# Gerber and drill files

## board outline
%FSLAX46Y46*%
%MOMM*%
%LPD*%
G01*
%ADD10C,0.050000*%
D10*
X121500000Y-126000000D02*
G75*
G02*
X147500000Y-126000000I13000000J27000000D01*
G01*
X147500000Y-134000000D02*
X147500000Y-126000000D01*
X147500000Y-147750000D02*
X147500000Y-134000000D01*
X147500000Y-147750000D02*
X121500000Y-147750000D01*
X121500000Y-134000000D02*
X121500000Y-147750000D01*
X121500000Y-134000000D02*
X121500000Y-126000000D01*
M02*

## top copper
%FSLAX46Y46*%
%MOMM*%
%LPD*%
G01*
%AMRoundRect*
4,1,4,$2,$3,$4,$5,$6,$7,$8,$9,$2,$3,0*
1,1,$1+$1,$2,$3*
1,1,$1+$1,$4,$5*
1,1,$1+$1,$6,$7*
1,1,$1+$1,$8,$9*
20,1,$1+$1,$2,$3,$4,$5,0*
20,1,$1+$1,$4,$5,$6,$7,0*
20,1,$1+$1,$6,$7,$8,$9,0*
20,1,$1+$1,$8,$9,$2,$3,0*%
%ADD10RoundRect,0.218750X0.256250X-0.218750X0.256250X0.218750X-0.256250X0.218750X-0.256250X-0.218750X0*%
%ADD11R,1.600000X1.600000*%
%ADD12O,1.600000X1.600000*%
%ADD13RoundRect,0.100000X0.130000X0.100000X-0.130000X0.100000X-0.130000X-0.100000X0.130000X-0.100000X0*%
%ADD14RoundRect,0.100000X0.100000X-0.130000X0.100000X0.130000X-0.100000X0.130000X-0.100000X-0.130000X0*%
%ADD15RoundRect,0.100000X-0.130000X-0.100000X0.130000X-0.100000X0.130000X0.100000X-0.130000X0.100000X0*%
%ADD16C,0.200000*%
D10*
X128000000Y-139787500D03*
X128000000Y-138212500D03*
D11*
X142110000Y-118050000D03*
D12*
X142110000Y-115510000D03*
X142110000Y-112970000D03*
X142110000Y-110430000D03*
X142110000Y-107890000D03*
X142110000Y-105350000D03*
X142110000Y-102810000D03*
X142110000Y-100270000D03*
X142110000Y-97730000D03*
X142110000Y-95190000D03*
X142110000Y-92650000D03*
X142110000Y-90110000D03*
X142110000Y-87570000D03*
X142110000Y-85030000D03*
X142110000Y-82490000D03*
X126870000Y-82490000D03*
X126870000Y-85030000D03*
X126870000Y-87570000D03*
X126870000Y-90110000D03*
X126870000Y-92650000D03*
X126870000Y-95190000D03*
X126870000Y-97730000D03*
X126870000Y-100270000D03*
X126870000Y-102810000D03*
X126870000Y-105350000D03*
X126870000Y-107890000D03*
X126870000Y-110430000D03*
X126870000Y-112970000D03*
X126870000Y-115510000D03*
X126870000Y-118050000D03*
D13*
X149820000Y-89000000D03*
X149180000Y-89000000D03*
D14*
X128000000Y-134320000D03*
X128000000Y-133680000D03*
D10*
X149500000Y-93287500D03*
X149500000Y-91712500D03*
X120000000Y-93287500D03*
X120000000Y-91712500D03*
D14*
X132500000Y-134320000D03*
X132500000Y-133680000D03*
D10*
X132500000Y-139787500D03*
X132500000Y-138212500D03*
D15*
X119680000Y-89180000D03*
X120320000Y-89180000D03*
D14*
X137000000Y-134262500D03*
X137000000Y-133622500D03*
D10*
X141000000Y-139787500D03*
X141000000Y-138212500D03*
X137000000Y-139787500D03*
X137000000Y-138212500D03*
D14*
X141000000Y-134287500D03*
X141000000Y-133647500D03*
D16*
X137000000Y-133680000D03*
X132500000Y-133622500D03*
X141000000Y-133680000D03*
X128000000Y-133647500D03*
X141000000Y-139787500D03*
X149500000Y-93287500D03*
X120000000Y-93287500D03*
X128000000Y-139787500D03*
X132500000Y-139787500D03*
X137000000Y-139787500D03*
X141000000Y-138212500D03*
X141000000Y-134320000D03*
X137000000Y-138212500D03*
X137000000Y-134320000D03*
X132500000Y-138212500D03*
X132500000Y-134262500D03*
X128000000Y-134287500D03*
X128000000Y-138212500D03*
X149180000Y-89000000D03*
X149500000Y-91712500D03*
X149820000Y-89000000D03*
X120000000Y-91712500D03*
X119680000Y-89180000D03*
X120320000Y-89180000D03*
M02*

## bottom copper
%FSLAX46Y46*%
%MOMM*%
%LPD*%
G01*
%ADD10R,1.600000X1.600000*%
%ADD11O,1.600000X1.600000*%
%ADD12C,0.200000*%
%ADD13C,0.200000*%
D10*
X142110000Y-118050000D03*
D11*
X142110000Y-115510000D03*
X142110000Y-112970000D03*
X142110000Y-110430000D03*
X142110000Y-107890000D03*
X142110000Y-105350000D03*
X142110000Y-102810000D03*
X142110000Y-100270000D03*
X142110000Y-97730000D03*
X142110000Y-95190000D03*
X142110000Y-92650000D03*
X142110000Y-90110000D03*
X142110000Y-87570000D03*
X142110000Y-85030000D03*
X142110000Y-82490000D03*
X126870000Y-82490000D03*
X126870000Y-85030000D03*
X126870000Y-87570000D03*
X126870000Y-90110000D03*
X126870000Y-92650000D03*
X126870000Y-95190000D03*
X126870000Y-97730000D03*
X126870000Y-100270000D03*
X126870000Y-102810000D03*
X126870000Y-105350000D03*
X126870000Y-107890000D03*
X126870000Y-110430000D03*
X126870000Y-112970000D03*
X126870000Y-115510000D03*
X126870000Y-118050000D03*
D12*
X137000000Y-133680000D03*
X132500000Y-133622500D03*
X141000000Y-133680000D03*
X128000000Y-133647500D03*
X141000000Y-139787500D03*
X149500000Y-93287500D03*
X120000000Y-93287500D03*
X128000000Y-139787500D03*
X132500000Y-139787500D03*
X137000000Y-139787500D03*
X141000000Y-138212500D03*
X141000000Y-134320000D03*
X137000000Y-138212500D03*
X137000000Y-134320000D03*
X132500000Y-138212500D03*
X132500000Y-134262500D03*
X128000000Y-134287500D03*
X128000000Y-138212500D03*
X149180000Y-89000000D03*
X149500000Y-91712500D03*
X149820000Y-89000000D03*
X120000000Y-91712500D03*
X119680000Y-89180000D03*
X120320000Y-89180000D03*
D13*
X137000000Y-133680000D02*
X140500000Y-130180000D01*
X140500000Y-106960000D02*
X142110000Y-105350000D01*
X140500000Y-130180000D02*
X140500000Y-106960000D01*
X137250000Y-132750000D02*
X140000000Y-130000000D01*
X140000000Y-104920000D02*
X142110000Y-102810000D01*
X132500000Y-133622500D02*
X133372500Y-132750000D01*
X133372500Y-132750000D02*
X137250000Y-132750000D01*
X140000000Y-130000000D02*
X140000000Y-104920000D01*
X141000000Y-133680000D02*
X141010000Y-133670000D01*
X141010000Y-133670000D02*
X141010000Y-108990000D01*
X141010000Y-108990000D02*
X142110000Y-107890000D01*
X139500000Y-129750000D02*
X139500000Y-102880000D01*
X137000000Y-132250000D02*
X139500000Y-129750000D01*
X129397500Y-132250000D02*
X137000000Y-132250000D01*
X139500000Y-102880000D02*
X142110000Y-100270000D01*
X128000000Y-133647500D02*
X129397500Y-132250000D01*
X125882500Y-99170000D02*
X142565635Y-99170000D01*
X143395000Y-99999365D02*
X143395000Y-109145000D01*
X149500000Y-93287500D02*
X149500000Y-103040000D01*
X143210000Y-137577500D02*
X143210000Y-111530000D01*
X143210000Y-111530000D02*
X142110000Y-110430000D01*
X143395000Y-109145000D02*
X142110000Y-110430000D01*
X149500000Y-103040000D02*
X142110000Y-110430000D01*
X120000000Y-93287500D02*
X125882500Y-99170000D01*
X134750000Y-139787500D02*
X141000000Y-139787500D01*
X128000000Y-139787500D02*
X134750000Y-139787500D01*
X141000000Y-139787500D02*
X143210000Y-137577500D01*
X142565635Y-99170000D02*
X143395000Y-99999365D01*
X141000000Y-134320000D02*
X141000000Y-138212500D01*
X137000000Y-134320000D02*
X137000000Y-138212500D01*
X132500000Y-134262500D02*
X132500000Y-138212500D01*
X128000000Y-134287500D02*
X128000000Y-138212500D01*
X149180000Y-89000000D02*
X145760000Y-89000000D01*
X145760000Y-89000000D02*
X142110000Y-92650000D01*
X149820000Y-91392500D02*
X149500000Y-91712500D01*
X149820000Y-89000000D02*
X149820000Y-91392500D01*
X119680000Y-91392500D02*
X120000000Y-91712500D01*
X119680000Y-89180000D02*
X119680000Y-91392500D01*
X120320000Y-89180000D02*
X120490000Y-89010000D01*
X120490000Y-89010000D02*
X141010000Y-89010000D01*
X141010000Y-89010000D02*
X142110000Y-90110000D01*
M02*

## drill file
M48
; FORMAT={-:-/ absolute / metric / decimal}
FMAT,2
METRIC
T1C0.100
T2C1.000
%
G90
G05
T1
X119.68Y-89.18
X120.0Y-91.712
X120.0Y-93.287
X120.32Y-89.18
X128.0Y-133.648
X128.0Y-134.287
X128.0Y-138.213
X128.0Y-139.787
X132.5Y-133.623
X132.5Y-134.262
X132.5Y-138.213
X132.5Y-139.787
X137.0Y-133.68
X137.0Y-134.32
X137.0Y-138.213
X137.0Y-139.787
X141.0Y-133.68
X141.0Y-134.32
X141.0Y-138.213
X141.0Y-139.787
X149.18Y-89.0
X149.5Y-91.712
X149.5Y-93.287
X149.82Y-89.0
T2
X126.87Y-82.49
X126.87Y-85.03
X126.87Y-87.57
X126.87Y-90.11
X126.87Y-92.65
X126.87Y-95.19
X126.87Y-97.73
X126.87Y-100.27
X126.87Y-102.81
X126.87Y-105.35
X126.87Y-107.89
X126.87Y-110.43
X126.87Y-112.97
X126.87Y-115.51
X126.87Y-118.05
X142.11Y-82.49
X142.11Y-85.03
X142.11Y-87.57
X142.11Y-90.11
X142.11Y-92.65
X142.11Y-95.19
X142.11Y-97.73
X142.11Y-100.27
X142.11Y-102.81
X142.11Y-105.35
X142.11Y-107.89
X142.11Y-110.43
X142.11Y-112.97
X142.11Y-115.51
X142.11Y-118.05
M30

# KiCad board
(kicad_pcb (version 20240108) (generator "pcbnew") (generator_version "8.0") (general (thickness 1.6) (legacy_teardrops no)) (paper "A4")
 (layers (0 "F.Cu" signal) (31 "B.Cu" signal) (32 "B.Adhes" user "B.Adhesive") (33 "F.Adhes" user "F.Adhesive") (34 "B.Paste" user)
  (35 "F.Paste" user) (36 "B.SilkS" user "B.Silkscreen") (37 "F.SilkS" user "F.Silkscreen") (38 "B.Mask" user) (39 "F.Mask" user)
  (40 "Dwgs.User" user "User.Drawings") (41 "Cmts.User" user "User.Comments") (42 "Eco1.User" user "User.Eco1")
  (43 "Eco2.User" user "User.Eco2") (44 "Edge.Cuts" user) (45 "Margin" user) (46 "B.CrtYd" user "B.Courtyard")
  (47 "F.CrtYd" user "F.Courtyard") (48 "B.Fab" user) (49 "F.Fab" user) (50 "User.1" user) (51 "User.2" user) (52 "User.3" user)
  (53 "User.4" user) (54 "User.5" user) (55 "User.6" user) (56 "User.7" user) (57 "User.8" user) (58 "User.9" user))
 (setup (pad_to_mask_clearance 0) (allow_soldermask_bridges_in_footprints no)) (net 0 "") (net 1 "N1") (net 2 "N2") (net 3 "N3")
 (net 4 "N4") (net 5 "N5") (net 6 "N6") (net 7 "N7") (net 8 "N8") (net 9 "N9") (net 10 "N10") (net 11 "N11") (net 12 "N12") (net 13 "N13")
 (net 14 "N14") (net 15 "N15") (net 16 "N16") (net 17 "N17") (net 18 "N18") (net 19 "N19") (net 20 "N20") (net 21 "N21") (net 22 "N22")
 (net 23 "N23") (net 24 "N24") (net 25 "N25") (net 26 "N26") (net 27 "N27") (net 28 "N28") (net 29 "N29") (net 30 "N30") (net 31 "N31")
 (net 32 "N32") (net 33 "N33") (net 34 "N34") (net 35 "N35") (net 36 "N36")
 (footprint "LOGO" (layer "F.Cu") (at 123.1 146.2)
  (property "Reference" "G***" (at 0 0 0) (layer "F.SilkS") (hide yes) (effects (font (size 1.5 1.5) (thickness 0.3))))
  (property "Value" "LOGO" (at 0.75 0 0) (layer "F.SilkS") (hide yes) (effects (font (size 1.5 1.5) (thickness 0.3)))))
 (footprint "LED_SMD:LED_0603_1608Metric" (layer "F.Cu") (at 128 139 90)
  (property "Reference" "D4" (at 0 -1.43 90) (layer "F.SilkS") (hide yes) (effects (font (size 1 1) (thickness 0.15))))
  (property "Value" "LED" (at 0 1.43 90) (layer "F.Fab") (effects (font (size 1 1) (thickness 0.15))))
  (pad "1" smd roundrect (at -0.7875 0 90) (size 0.875 0.95) (layers "F.Cu" "F.Paste" "F.Mask") (roundrect_rratio 0.25) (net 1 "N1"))
  (pad "2" smd roundrect (at 0.7875 0 90) (size 0.875 0.95) (layers "F.Cu" "F.Paste" "F.Mask") (roundrect_rratio 0.25) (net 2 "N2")))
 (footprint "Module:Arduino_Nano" (layer "F.Cu") (at 142.11 118.05 180)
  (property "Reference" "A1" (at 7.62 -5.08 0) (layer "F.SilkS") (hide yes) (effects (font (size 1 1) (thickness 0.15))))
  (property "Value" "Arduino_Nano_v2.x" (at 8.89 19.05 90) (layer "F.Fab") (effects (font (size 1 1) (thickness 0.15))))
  (pad "1" thru_hole rect (at 0 0 180) (size 1.6 1.6) (drill 1) (layers "*.Cu" "*.Mask") (remove_unused_layers no) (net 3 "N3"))
  (pad "2" thru_hole oval (at 0 2.54 180) (size 1.6 1.6) (drill 1) (layers "*.Cu" "*.Mask") (remove_unused_layers no) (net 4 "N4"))
  (pad "3" thru_hole oval (at 0 5.08 180) (size 1.6 1.6) (drill 1) (layers "*.Cu" "*.Mask") (remove_unused_layers no) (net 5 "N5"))
  (pad "4" thru_hole oval (at 0 7.62 180) (size 1.6 1.6) (drill 1) (layers "*.Cu" "*.Mask") (remove_unused_layers no) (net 1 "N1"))
  (pad "5" thru_hole oval (at 0 10.16 180) (size 1.6 1.6) (drill 1) (layers "*.Cu" "*.Mask") (remove_unused_layers no) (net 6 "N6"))
  (pad "6" thru_hole oval (at 0 12.7 180) (size 1.6 1.6) (drill 1) (layers "*.Cu" "*.Mask") (remove_unused_layers no) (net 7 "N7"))
  (pad "7" thru_hole oval (at 0 15.24 180) (size 1.6 1.6) (drill 1) (layers "*.Cu" "*.Mask") (remove_unused_layers no) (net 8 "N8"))
  (pad "8" thru_hole oval (at 0 17.78 180) (size 1.6 1.6) (drill 1) (layers "*.Cu" "*.Mask") (remove_unused_layers no) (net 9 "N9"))
  (pad "9" thru_hole oval (at 0 20.32 180) (size 1.6 1.6) (drill 1) (layers "*.Cu" "*.Mask") (remove_unused_layers no) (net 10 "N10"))
  (pad "10" thru_hole oval (at 0 22.86 180) (size 1.6 1.6) (drill 1) (layers "*.Cu" "*.Mask") (remove_unused_layers no) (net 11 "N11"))
  (pad "11" thru_hole oval (at 0 25.4 180) (size 1.6 1.6) (drill 1) (layers "*.Cu" "*.Mask") (remove_unused_layers no) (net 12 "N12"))
  (pad "12" thru_hole oval (at 0 27.94 180) (size 1.6 1.6) (drill 1) (layers "*.Cu" "*.Mask") (remove_unused_layers no) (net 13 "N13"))
  (pad "13" thru_hole oval (at 0 30.48 180) (size 1.6 1.6) (drill 1) (layers "*.Cu" "*.Mask") (remove_unused_layers no) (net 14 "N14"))
  (pad "14" thru_hole oval (at 0 33.02 180) (size 1.6 1.6) (drill 1) (layers "*.Cu" "*.Mask") (remove_unused_layers no) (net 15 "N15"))
  (pad "15" thru_hole oval (at 0 35.56 180) (size 1.6 1.6) (drill 1) (layers "*.Cu" "*.Mask") (remove_unused_layers no) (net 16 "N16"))
  (pad "16" thru_hole oval (at 15.24 35.56 180) (size 1.6 1.6) (drill 1) (layers "*.Cu" "*.Mask") (remove_unused_layers no) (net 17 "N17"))
  (pad "17" thru_hole oval (at 15.24 33.02 180) (size 1.6 1.6) (drill 1) (layers "*.Cu" "*.Mask") (remove_unused_layers no) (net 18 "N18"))
  (pad "18" thru_hole oval (at 15.24 30.48 180) (size 1.6 1.6) (drill 1) (layers "*.Cu" "*.Mask") (remove_unused_layers no) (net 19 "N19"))
  (pad "19" thru_hole oval (at 15.24 27.94 180) (size 1.6 1.6) (drill 1) (layers "*.Cu" "*.Mask") (remove_unused_layers no) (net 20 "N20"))
  (pad "20" thru_hole oval (at 15.24 25.4 180) (size 1.6 1.6) (drill 1) (layers "*.Cu" "*.Mask") (remove_unused_layers no) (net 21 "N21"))
  (pad "21" thru_hole oval (at 15.24 22.86 180) (size 1.6 1.6) (drill 1) (layers "*.Cu" "*.Mask") (remove_unused_layers no) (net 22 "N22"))
  (pad "22" thru_hole oval (at 15.24 20.32 180) (size 1.6 1.6) (drill 1) (layers "*.Cu" "*.Mask") (remove_unused_layers no) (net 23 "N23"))
  (pad "23" thru_hole oval (at 15.24 17.78 180) (size 1.6 1.6) (drill 1) (layers "*.Cu" "*.Mask") (remove_unused_layers no) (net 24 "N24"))
  (pad "24" thru_hole oval (at 15.24 15.24 180) (size 1.6 1.6) (drill 1) (layers "*.Cu" "*.Mask") (remove_unused_layers no) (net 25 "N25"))
  (pad "25" thru_hole oval (at 15.24 12.7 180) (size 1.6 1.6) (drill 1) (layers "*.Cu" "*.Mask") (remove_unused_layers no) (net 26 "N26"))
  (pad "26" thru_hole oval (at 15.24 10.16 180) (size 1.6 1.6) (drill 1) (layers "*.Cu" "*.Mask") (remove_unused_layers no) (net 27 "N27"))
  (pad "27" thru_hole oval (at 15.24 7.62 180) (size 1.6 1.6) (drill 1) (layers "*.Cu" "*.Mask") (remove_unused_layers no) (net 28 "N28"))
  (pad "28" thru_hole oval (at 15.24 5.08 180) (size 1.6 1.6) (drill 1) (layers "*.Cu" "*.Mask") (remove_unused_layers no) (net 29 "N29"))
  (pad "29" thru_hole oval (at 15.24 2.54 180) (size 1.6 1.6) (drill 1) (layers "*.Cu" "*.Mask") (remove_unused_layers no) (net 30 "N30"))
  (pad "30" thru_hole oval (at 15.24 0 180) (size 1.6 1.6) (drill 1) (layers "*.Cu" "*.Mask") (remove_unused_layers no) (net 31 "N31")))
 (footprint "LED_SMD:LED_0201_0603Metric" (layer "F.Cu") (at 149.5 89 180)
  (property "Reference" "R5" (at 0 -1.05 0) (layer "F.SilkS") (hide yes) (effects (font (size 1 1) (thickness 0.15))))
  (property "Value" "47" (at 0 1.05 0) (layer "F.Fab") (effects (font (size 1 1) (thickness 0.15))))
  (pad "" smd roundrect (at -0.345 0 180) (size 0.318 0.36) (layers "F.Paste") (roundrect_rratio 0.25))
  (pad "" smd roundrect (at 0.345 0 180) (size 0.318 0.36) (layers "F.Paste") (roundrect_rratio 0.25))
  (pad "1" smd roundrect (at -0.32 0 180) (size 0.46 0.4) (layers "F.Cu" "F.Mask") (roundrect_rratio 0.25) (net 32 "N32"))
  (pad "2" smd roundrect (at 0.32 0 180) (size 0.46 0.4) (layers "F.Cu" "F.Mask") (roundrect_rratio 0.25) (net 12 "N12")))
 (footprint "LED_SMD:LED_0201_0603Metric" (layer "F.Cu") (at 128 134 90)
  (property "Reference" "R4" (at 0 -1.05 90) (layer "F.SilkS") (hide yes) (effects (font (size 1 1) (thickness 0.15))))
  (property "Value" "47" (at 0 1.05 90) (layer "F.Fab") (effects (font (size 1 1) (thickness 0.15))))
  (pad "" smd roundrect (at -0.345 0 90) (size 0.318 0.36) (layers "F.Paste") (roundrect_rratio 0.25))
  (pad "" smd roundrect (at 0.345 0 90) (size 0.318 0.36) (layers "F.Paste") (roundrect_rratio 0.25))
  (pad "1" smd roundrect (at -0.32 0 90) (size 0.46 0.4) (layers "F.Cu" "F.Mask") (roundrect_rratio 0.25) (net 2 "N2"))
  (pad "2" smd roundrect (at 0.32 0 90) (size 0.46 0.4) (layers "F.Cu" "F.Mask") (roundrect_rratio 0.25) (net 9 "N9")))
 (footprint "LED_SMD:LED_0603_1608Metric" (layer "F.Cu") (at 149.5 92.5 90)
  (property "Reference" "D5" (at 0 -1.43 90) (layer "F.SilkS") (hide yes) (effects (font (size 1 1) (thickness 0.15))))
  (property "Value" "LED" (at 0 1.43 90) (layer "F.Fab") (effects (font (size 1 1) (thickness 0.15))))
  (pad "1" smd roundrect (at -0.7875 0 90) (size 0.875 0.95) (layers "F.Cu" "F.Paste" "F.Mask") (roundrect_rratio 0.25) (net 1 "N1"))
  (pad "2" smd roundrect (at 0.7875 0 90) (size 0.875 0.95) (layers "F.Cu" "F.Paste" "F.Mask") (roundrect_rratio 0.25) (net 32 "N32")))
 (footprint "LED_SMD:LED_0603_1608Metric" (layer "F.Cu") (at 120 92.5 90)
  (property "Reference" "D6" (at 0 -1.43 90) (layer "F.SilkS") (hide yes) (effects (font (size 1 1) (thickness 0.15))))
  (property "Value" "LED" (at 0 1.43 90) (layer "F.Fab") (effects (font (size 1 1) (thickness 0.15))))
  (pad "1" smd roundrect (at -0.7875 0 90) (size 0.875 0.95) (layers "F.Cu" "F.Paste" "F.Mask") (roundrect_rratio 0.25) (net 1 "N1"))
  (pad "2" smd roundrect (at 0.7875 0 90) (size 0.875 0.95) (layers "F.Cu" "F.Paste" "F.Mask") (roundrect_rratio 0.25) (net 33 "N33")))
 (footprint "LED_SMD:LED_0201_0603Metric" (layer "F.Cu") (at 132.5 134 90)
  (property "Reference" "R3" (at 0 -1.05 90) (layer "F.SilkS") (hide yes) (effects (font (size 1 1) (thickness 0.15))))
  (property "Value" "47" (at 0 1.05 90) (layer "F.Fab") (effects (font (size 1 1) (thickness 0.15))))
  (pad "" smd roundrect (at -0.345 0 90) (size 0.318 0.36) (layers "F.Paste") (roundrect_rratio 0.25))
  (pad "" smd roundrect (at 0.345 0 90) (size 0.318 0.36) (layers "F.Paste") (roundrect_rratio 0.25))
  (pad "1" smd roundrect (at -0.32 0 90) (size 0.46 0.4) (layers "F.Cu" "F.Mask") (roundrect_rratio 0.25) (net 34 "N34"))
  (pad "2" smd roundrect (at 0.32 0 90) (size 0.46 0.4) (layers "F.Cu" "F.Mask") (roundrect_rratio 0.25) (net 8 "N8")))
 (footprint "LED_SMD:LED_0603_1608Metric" (layer "F.Cu") (at 132.5 139 90)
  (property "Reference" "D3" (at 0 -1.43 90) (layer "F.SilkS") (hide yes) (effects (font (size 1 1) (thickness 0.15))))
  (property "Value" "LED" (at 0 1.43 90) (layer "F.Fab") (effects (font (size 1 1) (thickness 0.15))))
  (pad "1" smd roundrect (at -0.7875 0 90) (size 0.875 0.95) (layers "F.Cu" "F.Paste" "F.Mask") (roundrect_rratio 0.25) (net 1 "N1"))
  (pad "2" smd roundrect (at 0.7875 0 90) (size 0.875 0.95) (layers "F.Cu" "F.Paste" "F.Mask") (roundrect_rratio 0.25) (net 34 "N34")))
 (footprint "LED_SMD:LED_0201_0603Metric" (layer "F.Cu") (at 120 89.18)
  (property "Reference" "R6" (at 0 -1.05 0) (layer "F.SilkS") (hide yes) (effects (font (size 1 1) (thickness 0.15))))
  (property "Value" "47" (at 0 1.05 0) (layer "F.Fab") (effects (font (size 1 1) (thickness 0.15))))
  (pad "" smd roundrect (at -0.345 0) (size 0.318 0.36) (layers "F.Paste") (roundrect_rratio 0.25))
  (pad "" smd roundrect (at 0.345 0) (size 0.318 0.36) (layers "F.Paste") (roundrect_rratio 0.25))
  (pad "1" smd roundrect (at -0.32 0) (size 0.46 0.4) (layers "F.Cu" "F.Mask") (roundrect_rratio 0.25) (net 33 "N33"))
  (pad "2" smd roundrect (at 0.32 0) (size 0.46 0.4) (layers "F.Cu" "F.Mask") (roundrect_rratio 0.25) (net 13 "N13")))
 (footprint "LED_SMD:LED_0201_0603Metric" (layer "F.Cu") (at 137 133.9425 90)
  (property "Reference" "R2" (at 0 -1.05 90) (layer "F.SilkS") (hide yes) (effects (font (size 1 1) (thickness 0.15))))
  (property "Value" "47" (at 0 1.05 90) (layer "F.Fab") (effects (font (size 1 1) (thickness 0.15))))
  (pad "" smd roundrect (at -0.345 0 90) (size 0.318 0.36) (layers "F.Paste") (roundrect_rratio 0.25))
  (pad "" smd roundrect (at 0.345 0 90) (size 0.318 0.36) (layers "F.Paste") (roundrect_rratio 0.25))
  (pad "1" smd roundrect (at -0.32 0 90) (size 0.46 0.4) (layers "F.Cu" "F.Mask") (roundrect_rratio 0.25) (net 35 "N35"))
  (pad "2" smd roundrect (at 0.32 0 90) (size 0.46 0.4) (layers "F.Cu" "F.Mask") (roundrect_rratio 0.25) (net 7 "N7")))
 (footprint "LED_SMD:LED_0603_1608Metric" (layer "F.Cu") (at 141 139 90)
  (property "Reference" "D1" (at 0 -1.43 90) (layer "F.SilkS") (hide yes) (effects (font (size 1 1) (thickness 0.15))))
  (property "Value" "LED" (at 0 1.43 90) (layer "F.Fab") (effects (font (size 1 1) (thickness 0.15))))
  (pad "1" smd roundrect (at -0.7875 0 90) (size 0.875 0.95) (layers "F.Cu" "F.Paste" "F.Mask") (roundrect_rratio 0.25) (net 1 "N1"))
  (pad "2" smd roundrect (at 0.7875 0 90) (size 0.875 0.95) (layers "F.Cu" "F.Paste" "F.Mask") (roundrect_rratio 0.25) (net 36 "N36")))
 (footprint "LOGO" (layer "F.Cu") (at 134.5 115.75 90)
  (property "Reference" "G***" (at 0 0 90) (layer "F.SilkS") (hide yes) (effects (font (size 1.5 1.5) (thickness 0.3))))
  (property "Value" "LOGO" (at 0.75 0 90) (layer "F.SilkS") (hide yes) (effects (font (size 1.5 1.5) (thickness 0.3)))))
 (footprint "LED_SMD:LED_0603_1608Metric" (layer "F.Cu") (at 137 139 90)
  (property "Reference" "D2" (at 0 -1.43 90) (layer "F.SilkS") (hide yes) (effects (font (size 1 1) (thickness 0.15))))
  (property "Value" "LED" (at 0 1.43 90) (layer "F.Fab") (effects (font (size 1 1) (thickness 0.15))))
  (pad "1" smd roundrect (at -0.7875 0 90) (size 0.875 0.95) (layers "F.Cu" "F.Paste" "F.Mask") (roundrect_rratio 0.25) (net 1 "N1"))
  (pad "2" smd roundrect (at 0.7875 0 90) (size 0.875 0.95) (layers "F.Cu" "F.Paste" "F.Mask") (roundrect_rratio 0.25) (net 35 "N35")))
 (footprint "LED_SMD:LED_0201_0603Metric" (layer "F.Cu") (at 141 133.9675 90)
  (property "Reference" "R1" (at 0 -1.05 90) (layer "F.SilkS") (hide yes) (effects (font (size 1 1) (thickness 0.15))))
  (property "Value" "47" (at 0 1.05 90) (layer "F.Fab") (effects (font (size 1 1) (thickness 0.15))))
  (pad "" smd roundrect (at -0.345 0 90) (size 0.318 0.36) (layers "F.Paste") (roundrect_rratio 0.25))
  (pad "" smd roundrect (at 0.345 0 90) (size 0.318 0.36) (layers "F.Paste") (roundrect_rratio 0.25))
  (pad "1" smd roundrect (at -0.32 0 90) (size 0.46 0.4) (layers "F.Cu" "F.Mask") (roundrect_rratio 0.25) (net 36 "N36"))
  (pad "2" smd roundrect (at 0.32 0 90) (size 0.46 0.4) (layers "F.Cu" "F.Mask") (roundrect_rratio 0.25) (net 6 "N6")))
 (gr_arc (start 121.5 126) (mid 134.5 69.033352) (end 147.5 126) (stroke (width 0.05) (type default)) (layer "Edge.Cuts"))
 (gr_line (start 147.5 134) (end 147.5 126) (stroke (width 0.05) (type default)) (layer "Edge.Cuts"))
 (gr_line (start 147.5 147.75) (end 147.5 134) (stroke (width 0.05) (type default)) (layer "Edge.Cuts"))
 (gr_line (start 147.5 147.75) (end 121.5 147.75) (stroke (width 0.05) (type default)) (layer "Edge.Cuts"))
 (gr_line (start 121.5 134) (end 121.5 147.75) (stroke (width 0.05) (type default)) (layer "Edge.Cuts"))
 (gr_line (start 121.5 134) (end 121.5 126) (stroke (width 0.05) (type default)) (layer "Edge.Cuts"))
 (via (at 137 133.68) (size 0.2) (drill 0.1) (layers "F.Cu" "B.Cu") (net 7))
 (segment (start 137 133.68) (end 140.5 130.18) (width 0.2) (layer "B.Cu") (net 7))
 (segment (start 140.5 106.96) (end 142.11 105.35) (width 0.2) (layer "B.Cu") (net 7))
 (segment (start 140.5 130.18) (end 140.5 106.96) (width 0.2) (layer "B.Cu") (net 7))
 (via (at 132.5 133.6225) (size 0.2) (drill 0.1) (layers "F.Cu" "B.Cu") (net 8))
 (segment (start 137.25 132.75) (end 140 130) (width 0.2) (layer "B.Cu") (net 8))
 (segment (start 140 104.92) (end 142.11 102.81) (width 0.2) (layer "B.Cu") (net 8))
 (segment (start 132.5 133.6225) (end 133.3725 132.75) (width 0.2) (layer "B.Cu") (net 8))
 (segment (start 133.3725 132.75) (end 137.25 132.75) (width 0.2) (layer "B.Cu") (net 8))
 (segment (start 140 130) (end 140 104.92) (width 0.2) (layer "B.Cu") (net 8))
 (via (at 141 133.68) (size 0.2) (drill 0.1) (layers "F.Cu" "B.Cu") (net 6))
 (segment (start 141 133.68) (end 141.01 133.67) (width 0.2) (layer "B.Cu") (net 6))
 (segment (start 141.01 133.67) (end 141.01 108.99) (width 0.2) (layer "B.Cu") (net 6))
 (segment (start 141.01 108.99) (end 142.11 107.89) (width 0.2) (layer "B.Cu") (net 6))
 (via (at 128 133.6475) (size 0.2) (drill 0.1) (layers "F.Cu" "B.Cu") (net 9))
 (segment (start 139.5 129.75) (end 139.5 102.88) (width 0.2) (layer "B.Cu") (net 9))
 (segment (start 137 132.25) (end 139.5 129.75) (width 0.2) (layer "B.Cu") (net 9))
 (segment (start 129.3975 132.25) (end 137 132.25) (width 0.2) (layer "B.Cu") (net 9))
 (segment (start 139.5 102.88) (end 142.11 100.27) (width 0.2) (layer "B.Cu") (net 9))
 (segment (start 128 133.6475) (end 129.3975 132.25) (width 0.2) (layer "B.Cu") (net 9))
 (via (at 141 139.7875) (size 0.2) (drill 0.1) (layers "F.Cu" "B.Cu") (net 1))
 (via (at 149.5 93.2875) (size 0.2) (drill 0.1) (layers "F.Cu" "B.Cu") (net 1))
 (via (at 120 93.2875) (size 0.2) (drill 0.1) (layers "F.Cu" "B.Cu") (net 1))
 (via (at 128 139.7875) (size 0.2) (drill 0.1) (layers "F.Cu" "B.Cu") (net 1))
 (via (at 132.5 139.7875) (size 0.2) (drill 0.1) (layers "F.Cu" "B.Cu") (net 1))
 (via (at 137 139.7875) (size 0.2) (drill 0.1) (layers "F.Cu" "B.Cu") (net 1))
 (segment (start 125.8825 99.17) (end 142.565635 99.17) (width 0.2) (layer "B.Cu") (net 1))
 (segment (start 143.395 99.999365) (end 143.395 109.145) (width 0.2) (layer "B.Cu") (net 1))
 (segment (start 149.5 93.2875) (end 149.5 103.04) (width 0.2) (layer "B.Cu") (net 1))
 (segment (start 143.21 137.5775) (end 143.21 111.53) (width 0.2) (layer "B.Cu") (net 1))
 (segment (start 143.21 111.53) (end 142.11 110.43) (width 0.2) (layer "B.Cu") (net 1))
 (segment (start 143.395 109.145) (end 142.11 110.43) (width 0.2) (layer "B.Cu") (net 1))
 (segment (start 149.5 103.04) (end 142.11 110.43) (width 0.2) (layer "B.Cu") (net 1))
 (segment (start 120 93.2875) (end 125.8825 99.17) (width 0.2) (layer "B.Cu") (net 1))
 (segment (start 134.75 139.7875) (end 141 139.7875) (width 0.2) (layer "B.Cu") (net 1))
 (segment (start 128 139.7875) (end 134.75 139.7875) (width 0.2) (layer "B.Cu") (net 1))
 (segment (start 141 139.7875) (end 143.21 137.5775) (width 0.2) (layer "B.Cu") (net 1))
 (segment (start 142.565635 99.17) (end 143.395 99.999365) (width 0.2) (layer "B.Cu") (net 1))
 (via (at 141 138.2125) (size 0.2) (drill 0.1) (layers "F.Cu" "B.Cu") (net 36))
 (via (at 141 134.32) (size 0.2) (drill 0.1) (layers "F.Cu" "B.Cu") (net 36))
 (segment (start 141 134.32) (end 141 138.2125) (width 0.2) (layer "B.Cu") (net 36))
 (via (at 137 138.2125) (size 0.2) (drill 0.1) (layers "F.Cu" "B.Cu") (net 35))
 (via (at 137 134.32) (size 0.2) (drill 0.1) (layers "F.Cu" "B.Cu") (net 35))
 (segment (start 137 134.32) (end 137 138.2125) (width 0.2) (layer "B.Cu") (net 35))
 (via (at 132.5 138.2125) (size 0.2) (drill 0.1) (layers "F.Cu" "B.Cu") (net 34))
 (via (at 132.5 134.2625) (size 0.2) (drill 0.1) (layers "F.Cu" "B.Cu") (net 34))
 (segment (start 132.5 134.2625) (end 132.5 138.2125) (width 0.2) (layer "B.Cu") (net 34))
 (via (at 128 134.2875) (size 0.2) (drill 0.1) (layers "F.Cu" "B.Cu") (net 2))
 (via (at 128 138.2125) (size 0.2) (drill 0.1) (layers "F.Cu" "B.Cu") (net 2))
 (segment (start 128 134.2875) (end 128 138.2125) (width 0.2) (layer "B.Cu") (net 2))
 (via (at 149.18 89) (size 0.2) (drill 0.1) (layers "F.Cu" "B.Cu") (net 12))
 (segment (start 149.18 89) (end 145.76 89) (width 0.2) (layer "B.Cu") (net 12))
 (segment (start 145.76 89) (end 142.11 92.65) (width 0.2) (layer "B.Cu") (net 12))
 (via (at 149.5 91.7125) (size 0.2) (drill 0.1) (layers "F.Cu" "B.Cu") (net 32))
 (via (at 149.82 89) (size 0.2) (drill 0.1) (layers "F.Cu" "B.Cu") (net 32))
 (segment (start 149.82 91.3925) (end 149.5 91.7125) (width 0.2) (layer "B.Cu") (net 32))
 (segment (start 149.82 89) (end 149.82 91.3925) (width 0.2) (layer "B.Cu") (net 32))
 (via (at 120 91.7125) (size 0.2) (drill 0.1) (layers "F.Cu" "B.Cu") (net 33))
 (via (at 119.68 89.18) (size 0.2) (drill 0.1) (layers "F.Cu" "B.Cu") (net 33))
 (segment (start 119.68 91.3925) (end 120 91.7125) (width 0.2) (layer "B.Cu") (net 33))
 (segment (start 119.68 89.18) (end 119.68 91.3925) (width 0.2) (layer "B.Cu") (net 33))
 (via (at 120.32 89.18) (size 0.2) (drill 0.1) (layers "F.Cu" "B.Cu") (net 13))
 (segment (start 120.32 89.18) (end 120.49 89.01) (width 0.2) (layer "B.Cu") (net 13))
 (segment (start 120.49 89.01) (end 141.01 89.01) (width 0.2) (layer "B.Cu") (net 13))
 (segment (start 141.01 89.01) (end 142.11 90.11) (width 0.2) (layer "B.Cu") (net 13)))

